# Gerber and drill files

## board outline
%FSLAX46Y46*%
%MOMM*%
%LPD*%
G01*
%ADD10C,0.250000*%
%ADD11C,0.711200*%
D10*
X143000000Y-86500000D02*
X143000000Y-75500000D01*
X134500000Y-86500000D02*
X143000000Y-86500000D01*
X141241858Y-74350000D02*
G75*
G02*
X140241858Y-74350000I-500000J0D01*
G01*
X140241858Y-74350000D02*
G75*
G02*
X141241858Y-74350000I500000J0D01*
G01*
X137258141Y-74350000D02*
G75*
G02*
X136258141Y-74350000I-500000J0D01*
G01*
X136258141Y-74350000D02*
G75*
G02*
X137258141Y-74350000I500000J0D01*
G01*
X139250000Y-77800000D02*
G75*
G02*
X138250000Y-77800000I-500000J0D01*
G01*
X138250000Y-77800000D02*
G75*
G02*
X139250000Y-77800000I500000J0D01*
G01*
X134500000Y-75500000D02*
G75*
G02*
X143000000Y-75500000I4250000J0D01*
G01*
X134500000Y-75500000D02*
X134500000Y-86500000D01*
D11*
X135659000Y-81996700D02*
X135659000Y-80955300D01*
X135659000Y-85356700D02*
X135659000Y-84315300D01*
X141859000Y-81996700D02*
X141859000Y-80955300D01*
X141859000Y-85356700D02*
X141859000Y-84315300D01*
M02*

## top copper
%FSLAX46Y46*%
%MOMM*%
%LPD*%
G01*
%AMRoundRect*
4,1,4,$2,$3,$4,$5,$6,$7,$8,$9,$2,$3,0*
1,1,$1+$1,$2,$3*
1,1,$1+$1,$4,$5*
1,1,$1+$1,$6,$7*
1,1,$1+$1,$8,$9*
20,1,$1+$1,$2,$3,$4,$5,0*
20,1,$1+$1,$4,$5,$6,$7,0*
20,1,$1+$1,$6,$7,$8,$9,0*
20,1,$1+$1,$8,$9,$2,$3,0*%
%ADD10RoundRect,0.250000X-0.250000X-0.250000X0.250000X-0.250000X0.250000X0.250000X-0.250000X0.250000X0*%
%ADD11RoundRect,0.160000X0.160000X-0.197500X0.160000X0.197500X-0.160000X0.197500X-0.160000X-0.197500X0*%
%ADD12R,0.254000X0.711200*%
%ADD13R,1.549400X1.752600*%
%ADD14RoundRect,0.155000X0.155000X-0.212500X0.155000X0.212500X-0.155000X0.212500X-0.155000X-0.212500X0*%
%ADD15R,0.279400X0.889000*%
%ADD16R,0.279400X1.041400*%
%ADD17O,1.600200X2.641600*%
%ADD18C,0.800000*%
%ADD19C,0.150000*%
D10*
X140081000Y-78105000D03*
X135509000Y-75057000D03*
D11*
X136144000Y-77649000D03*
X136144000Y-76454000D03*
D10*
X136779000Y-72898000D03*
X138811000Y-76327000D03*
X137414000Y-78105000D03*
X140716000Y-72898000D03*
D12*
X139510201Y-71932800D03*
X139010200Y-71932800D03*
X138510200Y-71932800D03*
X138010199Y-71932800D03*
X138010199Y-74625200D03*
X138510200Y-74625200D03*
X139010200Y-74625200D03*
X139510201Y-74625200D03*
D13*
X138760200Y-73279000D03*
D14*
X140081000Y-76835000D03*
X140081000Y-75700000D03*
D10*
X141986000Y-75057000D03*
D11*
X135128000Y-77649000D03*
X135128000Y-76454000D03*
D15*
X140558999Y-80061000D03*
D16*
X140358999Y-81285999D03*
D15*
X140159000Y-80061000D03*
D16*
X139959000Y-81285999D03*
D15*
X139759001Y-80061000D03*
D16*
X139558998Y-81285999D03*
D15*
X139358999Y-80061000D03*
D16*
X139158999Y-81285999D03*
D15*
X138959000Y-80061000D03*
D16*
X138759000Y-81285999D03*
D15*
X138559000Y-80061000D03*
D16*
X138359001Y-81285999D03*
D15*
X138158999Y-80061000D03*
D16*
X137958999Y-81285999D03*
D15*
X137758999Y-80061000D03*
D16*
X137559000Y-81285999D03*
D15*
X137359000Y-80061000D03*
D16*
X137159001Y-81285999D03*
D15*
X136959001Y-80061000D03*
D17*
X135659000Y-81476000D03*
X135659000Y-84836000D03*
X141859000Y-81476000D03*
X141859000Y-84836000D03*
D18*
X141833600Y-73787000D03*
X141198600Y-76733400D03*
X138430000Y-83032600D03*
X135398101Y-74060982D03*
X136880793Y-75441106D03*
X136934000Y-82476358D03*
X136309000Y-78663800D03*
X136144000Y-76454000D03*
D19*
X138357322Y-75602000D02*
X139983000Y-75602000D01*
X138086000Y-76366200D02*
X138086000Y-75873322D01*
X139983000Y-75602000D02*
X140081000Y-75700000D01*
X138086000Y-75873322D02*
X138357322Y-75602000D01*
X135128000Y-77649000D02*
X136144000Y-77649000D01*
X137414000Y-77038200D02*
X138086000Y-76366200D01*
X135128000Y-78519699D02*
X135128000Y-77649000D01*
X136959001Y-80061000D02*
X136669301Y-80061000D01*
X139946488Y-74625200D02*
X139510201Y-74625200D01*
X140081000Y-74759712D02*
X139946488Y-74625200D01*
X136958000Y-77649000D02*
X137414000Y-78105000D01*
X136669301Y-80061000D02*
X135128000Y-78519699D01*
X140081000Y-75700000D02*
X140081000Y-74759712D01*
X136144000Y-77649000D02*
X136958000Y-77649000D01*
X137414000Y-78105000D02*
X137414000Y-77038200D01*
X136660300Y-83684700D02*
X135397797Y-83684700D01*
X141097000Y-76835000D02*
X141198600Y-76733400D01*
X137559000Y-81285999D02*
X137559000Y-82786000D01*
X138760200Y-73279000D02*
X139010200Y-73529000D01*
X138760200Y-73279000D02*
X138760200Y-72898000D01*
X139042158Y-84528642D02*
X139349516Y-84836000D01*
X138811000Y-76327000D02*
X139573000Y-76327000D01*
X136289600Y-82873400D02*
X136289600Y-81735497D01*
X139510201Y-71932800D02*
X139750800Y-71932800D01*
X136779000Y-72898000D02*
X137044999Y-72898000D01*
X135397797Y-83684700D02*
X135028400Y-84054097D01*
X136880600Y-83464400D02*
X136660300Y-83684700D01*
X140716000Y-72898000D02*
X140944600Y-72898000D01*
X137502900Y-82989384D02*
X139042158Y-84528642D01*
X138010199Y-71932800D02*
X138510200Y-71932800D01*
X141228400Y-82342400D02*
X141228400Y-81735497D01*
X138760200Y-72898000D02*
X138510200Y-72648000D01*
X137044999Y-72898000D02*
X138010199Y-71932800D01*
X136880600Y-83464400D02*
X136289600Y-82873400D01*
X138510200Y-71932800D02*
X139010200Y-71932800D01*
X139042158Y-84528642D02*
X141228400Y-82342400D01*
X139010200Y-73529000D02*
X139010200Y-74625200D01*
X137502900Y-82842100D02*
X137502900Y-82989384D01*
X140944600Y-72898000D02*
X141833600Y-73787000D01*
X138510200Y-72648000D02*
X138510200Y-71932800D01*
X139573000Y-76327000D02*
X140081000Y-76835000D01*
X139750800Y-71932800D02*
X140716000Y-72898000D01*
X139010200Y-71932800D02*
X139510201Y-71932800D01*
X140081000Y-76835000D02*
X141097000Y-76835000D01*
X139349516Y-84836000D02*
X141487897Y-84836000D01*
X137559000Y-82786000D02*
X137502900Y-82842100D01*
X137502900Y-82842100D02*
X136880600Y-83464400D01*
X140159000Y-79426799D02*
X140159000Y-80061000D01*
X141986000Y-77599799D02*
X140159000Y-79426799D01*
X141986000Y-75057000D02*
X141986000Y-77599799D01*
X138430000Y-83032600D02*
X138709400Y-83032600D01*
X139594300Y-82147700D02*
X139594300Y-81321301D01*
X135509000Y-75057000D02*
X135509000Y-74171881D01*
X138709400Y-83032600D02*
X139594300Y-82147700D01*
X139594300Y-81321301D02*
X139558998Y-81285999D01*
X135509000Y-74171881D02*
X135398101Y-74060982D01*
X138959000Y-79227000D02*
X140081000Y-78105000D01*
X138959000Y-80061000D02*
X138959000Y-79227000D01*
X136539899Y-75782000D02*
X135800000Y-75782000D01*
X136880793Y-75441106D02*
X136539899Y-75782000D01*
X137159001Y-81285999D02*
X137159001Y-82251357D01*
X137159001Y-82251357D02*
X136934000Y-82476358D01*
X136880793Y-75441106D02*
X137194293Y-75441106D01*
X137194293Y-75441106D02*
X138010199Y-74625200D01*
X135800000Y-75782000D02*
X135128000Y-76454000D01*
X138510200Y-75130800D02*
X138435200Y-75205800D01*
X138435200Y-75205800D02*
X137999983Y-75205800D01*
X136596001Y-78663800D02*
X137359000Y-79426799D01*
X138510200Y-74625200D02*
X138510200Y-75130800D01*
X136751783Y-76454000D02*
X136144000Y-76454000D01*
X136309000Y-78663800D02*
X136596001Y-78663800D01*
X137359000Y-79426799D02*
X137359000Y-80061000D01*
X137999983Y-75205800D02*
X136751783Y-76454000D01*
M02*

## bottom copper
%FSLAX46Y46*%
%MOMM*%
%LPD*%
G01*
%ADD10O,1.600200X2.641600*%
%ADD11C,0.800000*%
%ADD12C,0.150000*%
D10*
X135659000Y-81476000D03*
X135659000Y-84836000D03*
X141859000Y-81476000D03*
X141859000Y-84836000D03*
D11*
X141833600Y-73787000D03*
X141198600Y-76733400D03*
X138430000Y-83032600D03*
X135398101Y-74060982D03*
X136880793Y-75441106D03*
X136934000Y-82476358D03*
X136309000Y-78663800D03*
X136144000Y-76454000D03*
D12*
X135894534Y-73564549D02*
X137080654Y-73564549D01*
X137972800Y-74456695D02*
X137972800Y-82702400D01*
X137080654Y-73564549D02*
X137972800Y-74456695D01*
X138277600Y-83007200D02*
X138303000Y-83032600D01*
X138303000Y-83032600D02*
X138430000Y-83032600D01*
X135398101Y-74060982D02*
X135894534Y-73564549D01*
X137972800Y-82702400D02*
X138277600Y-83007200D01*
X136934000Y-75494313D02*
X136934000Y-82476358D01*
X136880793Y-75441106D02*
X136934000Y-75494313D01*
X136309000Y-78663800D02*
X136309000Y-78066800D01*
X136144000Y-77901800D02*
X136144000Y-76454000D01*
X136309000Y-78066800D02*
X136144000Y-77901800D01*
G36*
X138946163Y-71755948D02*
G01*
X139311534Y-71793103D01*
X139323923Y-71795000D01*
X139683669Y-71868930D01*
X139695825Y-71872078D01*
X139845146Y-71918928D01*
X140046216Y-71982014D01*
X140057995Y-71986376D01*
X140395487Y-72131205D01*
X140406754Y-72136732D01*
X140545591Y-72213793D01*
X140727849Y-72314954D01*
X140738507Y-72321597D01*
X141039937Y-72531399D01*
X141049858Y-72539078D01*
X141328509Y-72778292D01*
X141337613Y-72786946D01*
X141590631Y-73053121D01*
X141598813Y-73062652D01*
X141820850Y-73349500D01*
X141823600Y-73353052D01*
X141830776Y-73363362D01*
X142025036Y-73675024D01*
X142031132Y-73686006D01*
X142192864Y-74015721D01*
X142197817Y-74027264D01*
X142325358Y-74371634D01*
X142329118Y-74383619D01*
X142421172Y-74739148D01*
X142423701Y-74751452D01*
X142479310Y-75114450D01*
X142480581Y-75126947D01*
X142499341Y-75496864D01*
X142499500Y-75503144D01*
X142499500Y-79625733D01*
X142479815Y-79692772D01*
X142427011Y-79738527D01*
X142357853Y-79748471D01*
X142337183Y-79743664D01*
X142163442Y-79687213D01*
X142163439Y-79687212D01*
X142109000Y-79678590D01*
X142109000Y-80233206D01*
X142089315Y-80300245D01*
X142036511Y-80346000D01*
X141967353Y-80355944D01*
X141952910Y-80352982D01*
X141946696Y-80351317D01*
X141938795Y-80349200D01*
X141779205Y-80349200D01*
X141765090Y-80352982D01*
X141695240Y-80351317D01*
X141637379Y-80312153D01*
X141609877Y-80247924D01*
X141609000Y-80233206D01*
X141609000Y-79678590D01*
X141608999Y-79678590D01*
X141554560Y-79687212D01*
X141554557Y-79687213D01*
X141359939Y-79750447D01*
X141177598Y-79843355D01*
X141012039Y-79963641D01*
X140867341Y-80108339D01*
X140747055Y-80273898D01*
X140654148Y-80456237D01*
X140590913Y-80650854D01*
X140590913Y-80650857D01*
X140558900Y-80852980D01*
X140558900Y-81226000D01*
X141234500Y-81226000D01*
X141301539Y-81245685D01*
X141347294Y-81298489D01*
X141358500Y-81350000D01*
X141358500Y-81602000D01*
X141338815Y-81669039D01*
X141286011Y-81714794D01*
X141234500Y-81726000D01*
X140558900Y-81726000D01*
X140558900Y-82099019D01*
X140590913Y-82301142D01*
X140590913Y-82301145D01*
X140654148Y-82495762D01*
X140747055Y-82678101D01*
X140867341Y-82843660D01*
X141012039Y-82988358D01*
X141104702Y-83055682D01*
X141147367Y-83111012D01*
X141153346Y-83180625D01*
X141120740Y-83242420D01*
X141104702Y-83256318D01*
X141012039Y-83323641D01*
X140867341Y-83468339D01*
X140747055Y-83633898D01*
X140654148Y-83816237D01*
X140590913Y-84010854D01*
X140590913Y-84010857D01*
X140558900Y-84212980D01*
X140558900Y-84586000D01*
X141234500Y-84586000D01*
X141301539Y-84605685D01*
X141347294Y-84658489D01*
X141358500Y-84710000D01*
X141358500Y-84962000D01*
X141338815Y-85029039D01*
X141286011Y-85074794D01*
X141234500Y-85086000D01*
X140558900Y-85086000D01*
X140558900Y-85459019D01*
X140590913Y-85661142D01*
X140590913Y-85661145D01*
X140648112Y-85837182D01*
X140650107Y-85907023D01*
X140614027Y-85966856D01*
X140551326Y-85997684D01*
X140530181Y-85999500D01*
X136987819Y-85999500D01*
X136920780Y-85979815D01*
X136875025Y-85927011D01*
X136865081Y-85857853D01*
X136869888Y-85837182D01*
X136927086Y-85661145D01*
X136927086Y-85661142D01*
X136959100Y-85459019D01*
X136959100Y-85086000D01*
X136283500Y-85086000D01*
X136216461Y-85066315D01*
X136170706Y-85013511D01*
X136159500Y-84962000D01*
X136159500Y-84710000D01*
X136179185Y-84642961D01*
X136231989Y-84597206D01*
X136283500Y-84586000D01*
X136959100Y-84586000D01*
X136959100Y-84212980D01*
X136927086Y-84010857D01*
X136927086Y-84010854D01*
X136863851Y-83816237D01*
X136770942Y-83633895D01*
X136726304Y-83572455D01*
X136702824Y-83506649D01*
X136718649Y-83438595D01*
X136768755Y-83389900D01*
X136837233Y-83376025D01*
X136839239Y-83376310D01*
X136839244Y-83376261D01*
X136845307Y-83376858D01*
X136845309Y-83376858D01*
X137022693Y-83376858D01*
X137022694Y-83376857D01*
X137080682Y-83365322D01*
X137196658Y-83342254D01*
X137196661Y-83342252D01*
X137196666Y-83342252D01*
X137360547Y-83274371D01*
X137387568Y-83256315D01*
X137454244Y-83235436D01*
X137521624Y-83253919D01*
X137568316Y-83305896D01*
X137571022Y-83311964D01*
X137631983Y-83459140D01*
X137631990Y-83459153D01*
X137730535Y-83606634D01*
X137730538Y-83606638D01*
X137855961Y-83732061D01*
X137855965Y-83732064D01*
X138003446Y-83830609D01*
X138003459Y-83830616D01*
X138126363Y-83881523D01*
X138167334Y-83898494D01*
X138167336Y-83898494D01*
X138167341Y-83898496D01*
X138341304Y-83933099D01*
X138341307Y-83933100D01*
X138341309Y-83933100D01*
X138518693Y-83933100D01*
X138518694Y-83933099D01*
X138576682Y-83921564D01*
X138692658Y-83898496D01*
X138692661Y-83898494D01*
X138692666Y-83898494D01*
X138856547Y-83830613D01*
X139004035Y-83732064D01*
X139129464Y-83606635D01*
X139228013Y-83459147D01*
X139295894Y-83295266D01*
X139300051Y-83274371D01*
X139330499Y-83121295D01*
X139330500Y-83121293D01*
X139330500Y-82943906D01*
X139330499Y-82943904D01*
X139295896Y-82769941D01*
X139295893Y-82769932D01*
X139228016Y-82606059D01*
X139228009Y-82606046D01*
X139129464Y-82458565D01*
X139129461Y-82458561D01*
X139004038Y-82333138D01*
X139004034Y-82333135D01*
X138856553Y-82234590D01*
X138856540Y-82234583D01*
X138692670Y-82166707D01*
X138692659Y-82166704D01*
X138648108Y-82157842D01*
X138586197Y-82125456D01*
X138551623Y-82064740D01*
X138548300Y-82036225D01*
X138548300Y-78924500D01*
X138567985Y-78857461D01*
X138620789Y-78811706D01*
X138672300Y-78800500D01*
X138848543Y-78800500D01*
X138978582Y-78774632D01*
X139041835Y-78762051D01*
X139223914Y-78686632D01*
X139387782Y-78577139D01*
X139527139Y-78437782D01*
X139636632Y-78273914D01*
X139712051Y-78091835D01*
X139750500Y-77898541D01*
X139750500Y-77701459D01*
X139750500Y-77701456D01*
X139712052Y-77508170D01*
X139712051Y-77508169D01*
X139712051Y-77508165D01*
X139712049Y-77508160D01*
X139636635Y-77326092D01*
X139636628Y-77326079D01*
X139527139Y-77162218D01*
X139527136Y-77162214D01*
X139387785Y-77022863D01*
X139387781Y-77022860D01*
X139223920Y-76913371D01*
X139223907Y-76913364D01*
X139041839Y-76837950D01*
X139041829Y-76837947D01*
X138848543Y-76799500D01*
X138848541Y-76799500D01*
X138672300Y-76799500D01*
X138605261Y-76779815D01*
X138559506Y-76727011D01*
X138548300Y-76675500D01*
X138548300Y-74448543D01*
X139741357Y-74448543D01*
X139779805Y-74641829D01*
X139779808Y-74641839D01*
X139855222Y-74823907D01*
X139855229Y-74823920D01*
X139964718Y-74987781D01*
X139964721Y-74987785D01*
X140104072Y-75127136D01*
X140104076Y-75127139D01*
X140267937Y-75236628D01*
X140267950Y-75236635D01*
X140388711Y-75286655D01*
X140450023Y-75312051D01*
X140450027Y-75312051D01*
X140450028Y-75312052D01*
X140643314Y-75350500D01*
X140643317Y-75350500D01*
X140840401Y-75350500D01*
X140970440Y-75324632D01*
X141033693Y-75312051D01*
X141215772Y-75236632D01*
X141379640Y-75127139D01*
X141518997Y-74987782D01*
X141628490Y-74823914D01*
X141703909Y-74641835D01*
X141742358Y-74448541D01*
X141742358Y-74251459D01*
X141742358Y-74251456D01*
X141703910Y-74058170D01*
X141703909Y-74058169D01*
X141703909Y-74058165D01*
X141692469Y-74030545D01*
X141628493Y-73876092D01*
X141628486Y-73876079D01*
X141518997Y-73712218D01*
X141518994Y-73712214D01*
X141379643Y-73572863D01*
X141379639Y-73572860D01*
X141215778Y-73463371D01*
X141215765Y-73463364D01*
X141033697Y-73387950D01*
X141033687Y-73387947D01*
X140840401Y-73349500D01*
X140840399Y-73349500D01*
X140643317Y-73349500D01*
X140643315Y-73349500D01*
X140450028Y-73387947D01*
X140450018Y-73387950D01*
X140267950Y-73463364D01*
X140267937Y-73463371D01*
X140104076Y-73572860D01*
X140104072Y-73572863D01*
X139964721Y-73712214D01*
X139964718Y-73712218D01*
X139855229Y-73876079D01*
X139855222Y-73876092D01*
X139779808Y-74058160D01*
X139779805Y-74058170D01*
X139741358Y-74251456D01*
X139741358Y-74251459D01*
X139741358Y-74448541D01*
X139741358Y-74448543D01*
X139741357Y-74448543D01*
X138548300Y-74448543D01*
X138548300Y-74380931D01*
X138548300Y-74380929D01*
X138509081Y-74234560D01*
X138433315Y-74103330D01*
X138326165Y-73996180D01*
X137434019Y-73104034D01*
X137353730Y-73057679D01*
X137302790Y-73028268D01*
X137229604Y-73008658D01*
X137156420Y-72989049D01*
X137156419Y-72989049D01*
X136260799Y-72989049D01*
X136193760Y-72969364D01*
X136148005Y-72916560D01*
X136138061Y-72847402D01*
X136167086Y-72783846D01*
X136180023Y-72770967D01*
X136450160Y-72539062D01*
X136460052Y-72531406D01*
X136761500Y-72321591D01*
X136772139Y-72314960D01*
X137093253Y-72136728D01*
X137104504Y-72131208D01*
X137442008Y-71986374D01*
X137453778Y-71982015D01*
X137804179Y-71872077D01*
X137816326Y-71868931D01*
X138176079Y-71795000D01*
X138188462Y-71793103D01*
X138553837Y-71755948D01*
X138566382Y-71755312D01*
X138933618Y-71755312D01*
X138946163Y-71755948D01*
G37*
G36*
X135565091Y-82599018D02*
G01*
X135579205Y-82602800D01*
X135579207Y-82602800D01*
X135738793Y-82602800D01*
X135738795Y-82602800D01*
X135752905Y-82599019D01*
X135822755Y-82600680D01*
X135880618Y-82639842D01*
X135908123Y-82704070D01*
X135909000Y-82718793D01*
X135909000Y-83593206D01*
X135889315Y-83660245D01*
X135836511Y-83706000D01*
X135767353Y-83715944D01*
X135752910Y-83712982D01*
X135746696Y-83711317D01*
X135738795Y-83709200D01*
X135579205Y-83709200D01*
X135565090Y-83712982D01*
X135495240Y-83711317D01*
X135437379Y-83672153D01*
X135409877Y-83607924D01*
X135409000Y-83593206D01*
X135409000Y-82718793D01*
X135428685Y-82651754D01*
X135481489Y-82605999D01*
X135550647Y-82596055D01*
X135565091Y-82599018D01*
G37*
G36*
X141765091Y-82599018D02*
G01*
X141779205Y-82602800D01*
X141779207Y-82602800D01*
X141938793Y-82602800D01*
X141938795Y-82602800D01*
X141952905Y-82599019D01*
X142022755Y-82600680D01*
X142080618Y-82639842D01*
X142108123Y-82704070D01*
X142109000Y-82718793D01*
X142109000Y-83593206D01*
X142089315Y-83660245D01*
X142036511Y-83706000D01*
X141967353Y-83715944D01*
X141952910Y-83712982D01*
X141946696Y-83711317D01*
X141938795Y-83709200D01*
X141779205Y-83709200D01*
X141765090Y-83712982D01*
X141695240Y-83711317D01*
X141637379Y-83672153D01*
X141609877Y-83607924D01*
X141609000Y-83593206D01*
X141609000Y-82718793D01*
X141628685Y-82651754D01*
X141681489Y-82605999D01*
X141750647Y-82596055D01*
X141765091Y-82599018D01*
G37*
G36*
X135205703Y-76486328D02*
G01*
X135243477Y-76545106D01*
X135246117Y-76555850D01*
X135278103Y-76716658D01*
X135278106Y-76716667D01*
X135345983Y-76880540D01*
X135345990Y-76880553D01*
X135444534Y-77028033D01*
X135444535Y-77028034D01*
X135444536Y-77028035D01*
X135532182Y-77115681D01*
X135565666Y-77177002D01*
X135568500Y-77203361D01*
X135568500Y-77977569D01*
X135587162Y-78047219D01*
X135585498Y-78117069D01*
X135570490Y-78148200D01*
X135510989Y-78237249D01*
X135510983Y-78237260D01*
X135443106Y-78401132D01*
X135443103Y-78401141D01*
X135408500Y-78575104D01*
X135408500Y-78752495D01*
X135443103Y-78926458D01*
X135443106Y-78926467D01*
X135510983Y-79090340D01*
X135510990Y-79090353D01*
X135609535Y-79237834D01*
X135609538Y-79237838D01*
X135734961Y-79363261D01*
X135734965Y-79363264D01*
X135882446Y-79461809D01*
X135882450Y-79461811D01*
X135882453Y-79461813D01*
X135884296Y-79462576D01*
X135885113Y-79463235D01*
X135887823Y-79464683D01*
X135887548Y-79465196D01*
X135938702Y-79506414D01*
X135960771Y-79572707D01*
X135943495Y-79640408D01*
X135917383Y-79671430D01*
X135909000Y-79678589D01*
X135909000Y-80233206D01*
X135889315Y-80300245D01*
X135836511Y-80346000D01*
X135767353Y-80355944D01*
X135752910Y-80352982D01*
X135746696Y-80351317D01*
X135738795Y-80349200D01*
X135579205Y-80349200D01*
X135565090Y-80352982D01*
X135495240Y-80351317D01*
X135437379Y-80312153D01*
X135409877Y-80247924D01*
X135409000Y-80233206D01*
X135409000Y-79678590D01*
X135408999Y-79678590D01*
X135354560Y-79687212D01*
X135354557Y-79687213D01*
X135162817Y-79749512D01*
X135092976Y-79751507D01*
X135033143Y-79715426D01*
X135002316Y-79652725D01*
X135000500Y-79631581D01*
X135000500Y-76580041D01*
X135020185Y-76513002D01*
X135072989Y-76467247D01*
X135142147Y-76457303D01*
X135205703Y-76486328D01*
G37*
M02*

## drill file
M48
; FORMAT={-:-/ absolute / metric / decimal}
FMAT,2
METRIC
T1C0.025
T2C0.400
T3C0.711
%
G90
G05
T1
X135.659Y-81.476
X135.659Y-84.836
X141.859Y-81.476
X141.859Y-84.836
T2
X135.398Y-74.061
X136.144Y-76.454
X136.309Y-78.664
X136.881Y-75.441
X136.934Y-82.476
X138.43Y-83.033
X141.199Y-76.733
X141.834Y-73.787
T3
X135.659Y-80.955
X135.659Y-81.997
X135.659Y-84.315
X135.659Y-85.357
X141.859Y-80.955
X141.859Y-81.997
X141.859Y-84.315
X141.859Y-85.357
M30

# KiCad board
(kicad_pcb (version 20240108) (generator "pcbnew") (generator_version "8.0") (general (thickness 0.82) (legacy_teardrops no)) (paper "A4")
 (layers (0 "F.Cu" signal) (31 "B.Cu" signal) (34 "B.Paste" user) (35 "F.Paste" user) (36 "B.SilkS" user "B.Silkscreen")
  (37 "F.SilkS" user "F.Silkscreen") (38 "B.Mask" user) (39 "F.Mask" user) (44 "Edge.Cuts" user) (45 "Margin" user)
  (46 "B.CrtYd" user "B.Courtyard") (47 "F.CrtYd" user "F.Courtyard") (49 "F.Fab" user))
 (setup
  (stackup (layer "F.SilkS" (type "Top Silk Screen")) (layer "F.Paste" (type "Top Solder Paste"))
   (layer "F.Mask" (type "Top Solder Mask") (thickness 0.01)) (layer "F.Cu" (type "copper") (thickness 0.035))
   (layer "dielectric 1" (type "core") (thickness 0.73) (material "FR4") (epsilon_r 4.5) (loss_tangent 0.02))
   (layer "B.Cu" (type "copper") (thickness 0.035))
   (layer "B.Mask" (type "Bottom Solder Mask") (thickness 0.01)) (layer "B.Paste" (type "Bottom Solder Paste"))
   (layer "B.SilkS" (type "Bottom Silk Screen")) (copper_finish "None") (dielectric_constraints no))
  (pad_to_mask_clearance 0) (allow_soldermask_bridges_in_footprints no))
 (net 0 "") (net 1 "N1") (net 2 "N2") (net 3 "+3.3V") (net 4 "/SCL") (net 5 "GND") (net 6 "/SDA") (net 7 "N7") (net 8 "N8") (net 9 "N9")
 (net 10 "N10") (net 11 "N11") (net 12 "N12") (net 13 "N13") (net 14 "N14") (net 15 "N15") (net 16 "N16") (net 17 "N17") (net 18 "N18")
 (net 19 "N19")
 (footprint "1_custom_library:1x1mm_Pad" (layer "F.Cu") (at 140.081 78.105)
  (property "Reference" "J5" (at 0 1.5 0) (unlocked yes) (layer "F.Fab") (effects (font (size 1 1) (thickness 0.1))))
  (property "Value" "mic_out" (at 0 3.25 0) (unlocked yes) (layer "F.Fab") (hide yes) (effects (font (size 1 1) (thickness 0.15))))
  (pad "1" smd roundrect (at 0 0) (size 1 1) (layers "F.Cu" "F.Mask") (roundrect_rratio 0.25) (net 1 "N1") (thermal_bridge_angle 45)))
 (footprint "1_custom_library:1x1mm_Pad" (layer "F.Cu") (at 135.509 75.057)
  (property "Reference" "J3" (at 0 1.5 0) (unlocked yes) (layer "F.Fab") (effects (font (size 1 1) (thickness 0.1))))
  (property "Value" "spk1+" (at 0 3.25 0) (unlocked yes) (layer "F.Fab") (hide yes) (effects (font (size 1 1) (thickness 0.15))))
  (pad "1" smd roundrect (at 0 0) (size 1 1) (layers "F.Cu" "F.Mask") (roundrect_rratio 0.25) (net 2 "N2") (thermal_bridge_angle 45)))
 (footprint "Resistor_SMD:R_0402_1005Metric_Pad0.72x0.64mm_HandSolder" (layer "F.Cu") (at 136.144 77.0515 90)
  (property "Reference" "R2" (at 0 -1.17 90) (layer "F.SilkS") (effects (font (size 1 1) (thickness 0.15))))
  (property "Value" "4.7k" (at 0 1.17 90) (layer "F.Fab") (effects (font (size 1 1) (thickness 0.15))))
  (pad "1" smd roundrect (at -0.5975 0 90) (size 0.715 0.64) (layers "F.Cu" "F.Paste" "F.Mask") (roundrect_rratio 0.25) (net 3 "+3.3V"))
  (pad "2" smd roundrect (at 0.5975 0 90) (size 0.715 0.64) (layers "F.Cu" "F.Paste" "F.Mask") (roundrect_rratio 0.25) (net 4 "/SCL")))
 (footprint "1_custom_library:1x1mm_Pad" (layer "F.Cu") (at 136.779 72.898)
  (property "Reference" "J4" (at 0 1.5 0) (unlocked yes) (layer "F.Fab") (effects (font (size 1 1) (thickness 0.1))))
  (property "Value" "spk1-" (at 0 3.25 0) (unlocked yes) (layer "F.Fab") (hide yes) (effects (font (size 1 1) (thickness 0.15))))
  (pad "1" smd roundrect (at 0 0) (size 1 1) (layers "F.Cu" "F.Mask") (roundrect_rratio 0.25) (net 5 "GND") (thermal_bridge_angle 45)))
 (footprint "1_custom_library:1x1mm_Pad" (layer "F.Cu") (at 138.811 76.327)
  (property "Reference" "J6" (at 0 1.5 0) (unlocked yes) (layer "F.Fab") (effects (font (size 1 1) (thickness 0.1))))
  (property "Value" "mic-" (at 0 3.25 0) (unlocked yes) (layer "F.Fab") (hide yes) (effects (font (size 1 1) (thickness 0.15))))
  (pad "1" smd roundrect (at 0 0) (size 1 1) (layers "F.Cu" "F.Mask") (roundrect_rratio 0.25) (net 5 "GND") (thermal_bridge_angle 45)))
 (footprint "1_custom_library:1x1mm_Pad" (layer "F.Cu") (at 137.414 78.105)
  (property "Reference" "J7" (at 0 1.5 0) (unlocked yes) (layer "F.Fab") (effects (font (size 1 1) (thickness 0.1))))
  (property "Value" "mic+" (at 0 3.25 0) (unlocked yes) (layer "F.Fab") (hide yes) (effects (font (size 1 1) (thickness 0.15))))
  (pad "1" smd roundrect (at 0 0) (size 1 1) (layers "F.Cu" "F.Mask") (roundrect_rratio 0.25) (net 3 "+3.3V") (thermal_bridge_angle 45)))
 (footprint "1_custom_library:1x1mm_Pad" (layer "F.Cu") (at 140.716 72.898)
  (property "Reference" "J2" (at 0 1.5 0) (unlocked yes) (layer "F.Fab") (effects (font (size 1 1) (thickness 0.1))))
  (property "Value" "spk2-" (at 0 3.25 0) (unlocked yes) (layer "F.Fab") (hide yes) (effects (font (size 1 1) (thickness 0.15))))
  (pad "1" smd roundrect (at 0 0) (size 1 1) (layers "F.Cu" "F.Mask") (roundrect_rratio 0.25) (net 5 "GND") (thermal_bridge_angle 45)))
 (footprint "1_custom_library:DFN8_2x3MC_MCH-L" (layer "F.Cu") (at 138.7602 73.279 -90)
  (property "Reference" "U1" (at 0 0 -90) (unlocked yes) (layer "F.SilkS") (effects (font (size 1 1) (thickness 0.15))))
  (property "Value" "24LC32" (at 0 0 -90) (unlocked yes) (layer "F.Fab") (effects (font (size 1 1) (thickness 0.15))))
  (pad "1" smd rect (at -1.3462 -0.750001 270) (size 0.7112 0.254) (layers "F.Cu" "F.Paste" "F.Mask") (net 5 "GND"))
  (pad "2" smd rect (at -1.3462 -0.25 270) (size 0.7112 0.254) (layers "F.Cu" "F.Paste" "F.Mask") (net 5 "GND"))
  (pad "3" smd rect (at -1.3462 0.25 270) (size 0.7112 0.254) (layers "F.Cu" "F.Paste" "F.Mask") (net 5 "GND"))
  (pad "4" smd rect (at -1.3462 0.750001 270) (size 0.7112 0.254) (layers "F.Cu" "F.Paste" "F.Mask") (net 5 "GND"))
  (pad "5" smd rect (at 1.3462 0.750001 270) (size 0.7112 0.254) (layers "F.Cu" "F.Paste" "F.Mask") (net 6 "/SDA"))
  (pad "6" smd rect (at 1.3462 0.25 270) (size 0.7112 0.254) (layers "F.Cu" "F.Paste" "F.Mask") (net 4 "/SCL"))
  (pad "7" smd rect (at 1.3462 -0.25 270) (size 0.7112 0.254) (layers "F.Cu" "F.Paste" "F.Mask") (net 5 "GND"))
  (pad "8" smd rect (at 1.3462 -0.750001 270) (size 0.7112 0.254) (layers "F.Cu" "F.Paste" "F.Mask") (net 3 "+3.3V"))
  (pad "9" smd rect (at 0 0 270) (size 1.7526 1.5494) (layers "F.Cu" "F.Paste" "F.Mask") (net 5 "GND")))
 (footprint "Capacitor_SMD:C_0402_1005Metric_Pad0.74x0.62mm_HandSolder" (layer "F.Cu") (at 140.081 76.2675 90)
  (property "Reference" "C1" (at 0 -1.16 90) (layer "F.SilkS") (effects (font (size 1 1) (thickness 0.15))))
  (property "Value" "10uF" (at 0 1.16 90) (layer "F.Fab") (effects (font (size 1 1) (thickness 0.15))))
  (pad "1" smd roundrect (at -0.5675 0 90) (size 0.735 0.62) (layers "F.Cu" "F.Paste" "F.Mask") (roundrect_rratio 0.25) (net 5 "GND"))
  (pad "2" smd roundrect (at 0.5675 0 90) (size 0.735 0.62) (layers "F.Cu" "F.Paste" "F.Mask") (roundrect_rratio 0.25) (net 3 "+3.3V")))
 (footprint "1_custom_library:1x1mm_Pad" (layer "F.Cu") (at 141.986 75.057)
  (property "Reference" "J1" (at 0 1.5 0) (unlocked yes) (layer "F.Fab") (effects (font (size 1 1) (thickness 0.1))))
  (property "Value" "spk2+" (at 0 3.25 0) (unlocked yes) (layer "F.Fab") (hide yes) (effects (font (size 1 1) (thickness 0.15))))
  (pad "1" smd roundrect (at 0 0) (size 1 1) (layers "F.Cu" "F.Mask") (roundrect_rratio 0.25) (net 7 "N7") (thermal_bridge_angle 45)))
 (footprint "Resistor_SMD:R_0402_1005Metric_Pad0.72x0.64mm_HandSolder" (layer "F.Cu") (at 135.128 77.0515 90)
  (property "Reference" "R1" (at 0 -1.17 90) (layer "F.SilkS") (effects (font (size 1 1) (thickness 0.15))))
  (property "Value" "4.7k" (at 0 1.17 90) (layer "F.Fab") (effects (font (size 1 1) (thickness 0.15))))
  (pad "1" smd roundrect (at -0.5975 0 90) (size 0.715 0.64) (layers "F.Cu" "F.Paste" "F.Mask") (roundrect_rratio 0.25) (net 3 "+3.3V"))
  (pad "2" smd roundrect (at 0.5975 0 90) (size 0.715 0.64) (layers "F.Cu" "F.Paste" "F.Mask") (roundrect_rratio 0.25) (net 6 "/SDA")))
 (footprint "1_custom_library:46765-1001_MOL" (layer "F.Cu") (at 138.759 83.3841)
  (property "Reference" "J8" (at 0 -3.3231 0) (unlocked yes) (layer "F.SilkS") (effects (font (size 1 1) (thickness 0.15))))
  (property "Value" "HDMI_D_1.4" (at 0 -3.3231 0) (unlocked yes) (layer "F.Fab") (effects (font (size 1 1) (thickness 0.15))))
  (fp_line (start -3.1 -1.3874) (end -3.1 -2.4288) (stroke (width 0.7112) (type solid)) (layer "Edge.Cuts"))
  (fp_line (start -3.1 1.9726) (end -3.1 0.9312) (stroke (width 0.7112) (type solid)) (layer "Edge.Cuts"))
  (fp_line (start 3.1 -1.3874) (end 3.1 -2.4288) (stroke (width 0.7112) (type solid)) (layer "Edge.Cuts"))
  (fp_line (start 3.1 1.9726) (end 3.1 0.9312) (stroke (width 0.7112) (type solid)) (layer "Edge.Cuts"))
  (pad "" np_thru_hole circle (at -3.1 -2.4288) (size 0.7112 0.7112) (drill 0.7112) (layers "*.Cu" "*.Mask"))
  (pad "" np_thru_hole circle (at -3.1 -1.3874) (size 0.7112 0.7112) (drill 0.7112) (layers "*.Cu" "*.Mask"))
  (pad "" np_thru_hole circle (at -3.1 0.9312) (size 0.7112 0.7112) (drill 0.7112) (layers "*.Cu" "*.Mask"))
  (pad "" np_thru_hole circle (at -3.1 1.9726) (size 0.7112 0.7112) (drill 0.7112) (layers "*.Cu" "*.Mask"))
  (pad "" np_thru_hole circle (at 3.1 -2.4288) (size 0.7112 0.7112) (drill 0.7112) (layers "*.Cu" "*.Mask"))
  (pad "" np_thru_hole circle (at 3.1 -1.3874) (size 0.7112 0.7112) (drill 0.7112) (layers "*.Cu" "*.Mask"))
  (pad "" np_thru_hole circle (at 3.1 0.9312) (size 0.7112 0.7112) (drill 0.7112) (layers "*.Cu" "*.Mask"))
  (pad "" np_thru_hole circle (at 3.1 1.9726) (size 0.7112 0.7112) (drill 0.7112) (layers "*.Cu" "*.Mask"))
  (pad "1" smd rect (at 1.799999 -3.3231) (size 0.2794 0.889) (layers "F.Cu" "F.Paste" "F.Mask") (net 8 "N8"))
  (pad "2" smd rect (at 1.599999 -2.098101) (size 0.2794 1.0414) (layers "F.Cu" "F.Paste" "F.Mask") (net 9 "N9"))
  (pad "3" smd rect (at 1.4 -3.3231) (size 0.2794 0.889) (layers "F.Cu" "F.Paste" "F.Mask") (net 7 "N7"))
  (pad "4" smd rect (at 1.2 -2.098101) (size 0.2794 1.0414) (layers "F.Cu" "F.Paste" "F.Mask") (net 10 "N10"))
  (pad "5" smd rect (at 1.000001 -3.3231) (size 0.2794 0.889) (layers "F.Cu" "F.Paste" "F.Mask") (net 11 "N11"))
  (pad "6" smd rect (at 0.799998 -2.098101) (size 0.2794 1.0414) (layers "F.Cu" "F.Paste" "F.Mask") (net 2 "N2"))
  (pad "7" smd rect (at 0.599999 -3.3231) (size 0.2794 0.889) (layers "F.Cu" "F.Paste" "F.Mask") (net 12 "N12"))
  (pad "8" smd rect (at 0.399999 -2.098101) (size 0.2794 1.0414) (layers "F.Cu" "F.Paste" "F.Mask") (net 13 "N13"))
  (pad "9" smd rect (at 0.2 -3.3231) (size 0.2794 0.889) (layers "F.Cu" "F.Paste" "F.Mask") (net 1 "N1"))
  (pad "10" smd rect (at 0 -2.098101) (size 0.2794 1.0414) (layers "F.Cu" "F.Paste" "F.Mask") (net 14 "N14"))
  (pad "11" smd rect (at -0.2 -3.3231) (size 0.2794 0.889) (layers "F.Cu" "F.Paste" "F.Mask") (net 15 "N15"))
  (pad "12" smd rect (at -0.399999 -2.098101) (size 0.2794 1.0414) (layers "F.Cu" "F.Paste" "F.Mask") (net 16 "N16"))
  (pad "13" smd rect (at -0.600001 -3.3231) (size 0.2794 0.889) (layers "F.Cu" "F.Paste" "F.Mask") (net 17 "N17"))
  (pad "14" smd rect (at -0.800001 -2.098101) (size 0.2794 1.0414) (layers "F.Cu" "F.Paste" "F.Mask") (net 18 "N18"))
  (pad "15" smd rect (at -1.000001 -3.3231) (size 0.2794 0.889) (layers "F.Cu" "F.Paste" "F.Mask") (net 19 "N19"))
  (pad "16" smd rect (at -1.2 -2.098101) (size 0.2794 1.0414) (layers "F.Cu" "F.Paste" "F.Mask") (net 5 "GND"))
  (pad "17" smd rect (at -1.4 -3.3231) (size 0.2794 0.889) (layers "F.Cu" "F.Paste" "F.Mask") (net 4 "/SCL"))
  (pad "18" smd rect (at -1.599999 -2.098101) (size 0.2794 1.0414) (layers "F.Cu" "F.Paste" "F.Mask") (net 6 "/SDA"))
  (pad "19" smd rect (at -1.799999 -3.3231) (size 0.2794 0.889) (layers "F.Cu" "F.Paste" "F.Mask") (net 3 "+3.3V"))
  (pad "SH" thru_hole oval (at -3.1 -1.9081 90) (size 2.6416 1.6002) (drill 0.0254) (layers "*.Cu" "*.Mask") (remove_unused_layers no)
   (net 5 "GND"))
  (pad "SH" thru_hole oval (at -3.1 1.4519 90) (size 2.6416 1.6002) (drill 0.0254) (layers "*.Cu" "*.Mask") (remove_unused_layers no)
   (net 5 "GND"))
  (pad "SH" thru_hole oval (at 3.1 -1.9081 90) (size 2.6416 1.6002) (drill 0.0254) (layers "*.Cu" "*.Mask") (remove_unused_layers no)
   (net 5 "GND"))
  (pad "SH" thru_hole oval (at 3.1 1.4519 90) (size 2.6416 1.6002) (drill 0.0254) (layers "*.Cu" "*.Mask") (remove_unused_layers no)
   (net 5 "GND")))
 (gr_line (start 143 86.5) (end 143 75.5) (stroke (width 0.25) (type default)) (layer "Edge.Cuts"))
 (gr_line (start 134.5 86.5) (end 143 86.5) (stroke (width 0.25) (type default)) (layer "Edge.Cuts"))
 (gr_circle (center 140.741858 74.35) (end 141.241858 74.35) (stroke (width 0.25) (type default)) (fill none) (layer "Edge.Cuts"))
 (gr_circle (center 136.758141 74.35) (end 137.258141 74.35) (stroke (width 0.25) (type default)) (fill none) (layer "Edge.Cuts"))
 (gr_circle (center 138.75 77.8) (end 139.25 77.8) (stroke (width 0.25) (type default)) (fill none) (layer "Edge.Cuts"))
 (gr_arc (start 134.5 75.5) (mid 138.75 71.25) (end 143 75.5) (stroke (width 0.25) (type default)) (layer "Edge.Cuts"))
 (gr_line (start 134.5 75.5) (end 134.5 86.5) (stroke (width 0.25) (type default)) (layer "Edge.Cuts"))
 (segment (start 138.357322 75.602) (end 139.983 75.602) (width 0.15) (layer "F.Cu") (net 3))
 (segment (start 138.086 76.3662) (end 138.086 75.873322) (width 0.15) (layer "F.Cu") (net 3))
 (segment (start 139.983 75.602) (end 140.081 75.7) (width 0.15) (layer "F.Cu") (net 3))
 (segment (start 138.086 75.873322) (end 138.357322 75.602) (width 0.15) (layer "F.Cu") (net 3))
 (segment (start 135.128 77.649) (end 136.144 77.649) (width 0.15) (layer "F.Cu") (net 3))
 (segment (start 137.414 77.0382) (end 138.086 76.3662) (width 0.15) (layer "F.Cu") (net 3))
 (segment (start 135.128 78.519699) (end 135.128 77.649) (width 0.15) (layer "F.Cu") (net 3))
 (segment (start 136.959001 80.061) (end 136.669301 80.061) (width 0.15) (layer "F.Cu") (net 3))
 (segment (start 139.946488 74.6252) (end 139.510201 74.6252) (width 0.15) (layer "F.Cu") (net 3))
 (segment (start 140.081 74.759712) (end 139.946488 74.6252) (width 0.15) (layer "F.Cu") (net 3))
 (segment (start 136.958 77.649) (end 137.414 78.105) (width 0.15) (layer "F.Cu") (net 3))
 (segment (start 136.669301 80.061) (end 135.128 78.519699) (width 0.15) (layer "F.Cu") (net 3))
 (segment (start 140.081 75.7) (end 140.081 74.759712) (width 0.15) (layer "F.Cu") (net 3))
 (segment (start 136.144 77.649) (end 136.958 77.649) (width 0.15) (layer "F.Cu") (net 3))
 (segment (start 137.414 78.105) (end 137.414 77.0382) (width 0.15) (layer "F.Cu") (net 3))
 (segment (start 136.6603 83.6847) (end 135.397797 83.6847) (width 0.15) (layer "F.Cu") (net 5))
 (segment (start 141.097 76.835) (end 141.1986 76.7334) (width 0.15) (layer "F.Cu") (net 5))
 (segment (start 137.559 81.285999) (end 137.559 82.786) (width 0.15) (layer "F.Cu") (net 5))
 (segment (start 138.7602 73.279) (end 139.0102 73.529) (width 0.15) (layer "F.Cu") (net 5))
 (segment (start 138.7602 73.279) (end 138.7602 72.898) (width 0.15) (layer "F.Cu") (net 5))
 (segment (start 139.042158 84.528642) (end 139.349516 84.836) (width 0.15) (layer "F.Cu") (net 5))
 (segment (start 138.811 76.327) (end 139.573 76.327) (width 0.15) (layer "F.Cu") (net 5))
 (segment (start 136.2896 82.8734) (end 136.2896 81.735497) (width 0.15) (layer "F.Cu") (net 5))
 (segment (start 139.510201 71.9328) (end 139.7508 71.9328) (width 0.15) (layer "F.Cu") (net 5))
 (segment (start 136.779 72.898) (end 137.044999 72.898) (width 0.15) (layer "F.Cu") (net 5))
 (segment (start 135.397797 83.6847) (end 135.0284 84.054097) (width 0.15) (layer "F.Cu") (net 5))
 (segment (start 136.8806 83.4644) (end 136.6603 83.6847) (width 0.15) (layer "F.Cu") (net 5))
 (segment (start 140.716 72.898) (end 140.9446 72.898) (width 0.15) (layer "F.Cu") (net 5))
 (segment (start 137.5029 82.989384) (end 139.042158 84.528642) (width 0.15) (layer "F.Cu") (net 5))
 (segment (start 138.010199 71.9328) (end 138.5102 71.9328) (width 0.15) (layer "F.Cu") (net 5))
 (segment (start 141.2284 82.3424) (end 141.2284 81.735497) (width 0.15) (layer "F.Cu") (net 5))
 (segment (start 138.7602 72.898) (end 138.5102 72.648) (width 0.15) (layer "F.Cu") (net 5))
 (segment (start 137.044999 72.898) (end 138.010199 71.9328) (width 0.15) (layer "F.Cu") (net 5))
 (segment (start 136.8806 83.4644) (end 136.2896 82.8734) (width 0.15) (layer "F.Cu") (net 5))
 (segment (start 138.5102 71.9328) (end 139.0102 71.9328) (width 0.15) (layer "F.Cu") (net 5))
 (segment (start 139.042158 84.528642) (end 141.2284 82.3424) (width 0.15) (layer "F.Cu") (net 5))
 (segment (start 139.0102 73.529) (end 139.0102 74.6252) (width 0.15) (layer "F.Cu") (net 5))
 (segment (start 137.5029 82.8421) (end 137.5029 82.989384) (width 0.15) (layer "F.Cu") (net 5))
 (segment (start 140.9446 72.898) (end 141.8336 73.787) (width 0.15) (layer "F.Cu") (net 5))
 (segment (start 138.5102 72.648) (end 138.5102 71.9328) (width 0.15) (layer "F.Cu") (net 5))
 (segment (start 139.573 76.327) (end 140.081 76.835) (width 0.15) (layer "F.Cu") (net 5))
 (segment (start 139.7508 71.9328) (end 140.716 72.898) (width 0.15) (layer "F.Cu") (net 5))
 (segment (start 139.0102 71.9328) (end 139.510201 71.9328) (width 0.15) (layer "F.Cu") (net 5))
 (segment (start 140.081 76.835) (end 141.097 76.835) (width 0.15) (layer "F.Cu") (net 5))
 (segment (start 139.349516 84.836) (end 141.487897 84.836) (width 0.15) (layer "F.Cu") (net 5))
 (segment (start 137.559 82.786) (end 137.5029 82.8421) (width 0.15) (layer "F.Cu") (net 5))
 (segment (start 137.5029 82.8421) (end 136.8806 83.4644) (width 0.15) (layer "F.Cu") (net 5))
 (via (at 141.8336 73.787) (size 0.8) (drill 0.4) (layers "F.Cu" "B.Cu") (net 5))
 (via (at 141.1986 76.7334) (size 0.8) (drill 0.4) (layers "F.Cu" "B.Cu") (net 5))
 (segment (start 140.159 79.426799) (end 140.159 80.061) (width 0.15) (layer "F.Cu") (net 7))
 (segment (start 141.986 77.599799) (end 140.159 79.426799) (width 0.15) (layer "F.Cu") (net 7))
 (segment (start 141.986 75.057) (end 141.986 77.599799) (width 0.15) (layer "F.Cu") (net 7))
 (segment (start 138.43 83.0326) (end 138.7094 83.0326) (width 0.15) (layer "F.Cu") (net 2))
 (segment (start 139.5943 82.1477) (end 139.5943 81.321301) (width 0.15) (layer "F.Cu") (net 2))
 (segment (start 135.509 75.057) (end 135.509 74.171881) (width 0.15) (layer "F.Cu") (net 2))
 (segment (start 138.7094 83.0326) (end 139.5943 82.1477) (width 0.15) (layer "F.Cu") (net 2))
 (segment (start 139.5943 81.321301) (end 139.558998 81.285999) (width 0.15) (layer "F.Cu") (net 2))
 (segment (start 135.509 74.171881) (end 135.398101 74.060982) (width 0.15) (layer "F.Cu") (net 2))
 (via (at 138.43 83.0326) (size 0.8) (drill 0.4) (layers "F.Cu" "B.Cu") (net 2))
 (via (at 135.398101 74.060982) (size 0.8) (drill 0.4) (layers "F.Cu" "B.Cu") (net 2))
 (segment (start 135.894534 73.564549) (end 137.080654 73.564549) (width 0.15) (layer "B.Cu") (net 2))
 (segment (start 137.9728 74.456695) (end 137.9728 82.7024) (width 0.15) (layer "B.Cu") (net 2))
 (segment (start 137.080654 73.564549) (end 137.9728 74.456695) (width 0.15) (layer "B.Cu") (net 2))
 (segment (start 138.2776 83.0072) (end 138.303 83.0326) (width 0.15) (layer "B.Cu") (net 2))
 (segment (start 138.303 83.0326) (end 138.43 83.0326) (width 0.15) (layer "B.Cu") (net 2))
 (segment (start 135.398101 74.060982) (end 135.894534 73.564549) (width 0.15) (layer "B.Cu") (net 2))
 (segment (start 137.9728 82.7024) (end 138.2776 83.0072) (width 0.15) (layer "B.Cu") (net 2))
 (segment (start 138.959 79.227) (end 140.081 78.105) (width 0.15) (layer "F.Cu") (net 1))
 (segment (start 138.959 80.061) (end 138.959 79.227) (width 0.15) (layer "F.Cu") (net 1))
 (segment (start 136.539899 75.782) (end 135.8 75.782) (width 0.15) (layer "F.Cu") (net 6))
 (segment (start 136.880793 75.441106) (end 136.539899 75.782) (width 0.15) (layer "F.Cu") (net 6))
 (segment (start 137.159001 81.285999) (end 137.159001 82.251357) (width 0.15) (layer "F.Cu") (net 6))
 (segment (start 137.159001 82.251357) (end 136.934 82.476358) (width 0.15) (layer "F.Cu") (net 6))
 (segment (start 136.880793 75.441106) (end 137.194293 75.441106) (width 0.15) (layer "F.Cu") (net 6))
 (segment (start 137.194293 75.441106) (end 138.010199 74.6252) (width 0.15) (layer "F.Cu") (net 6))
 (segment (start 135.8 75.782) (end 135.128 76.454) (width 0.15) (layer "F.Cu") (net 6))
 (via (at 136.880793 75.441106) (size 0.8) (drill 0.4) (layers "F.Cu" "B.Cu") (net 6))
 (via (at 136.934 82.476358) (size 0.8) (drill 0.4) (layers "F.Cu" "B.Cu") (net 6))
 (segment (start 136.934 75.494313) (end 136.934 82.476358) (width 0.15) (layer "B.Cu") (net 6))
 (segment (start 136.880793 75.441106) (end 136.934 75.494313) (width 0.15) (layer "B.Cu") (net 6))
 (segment (start 138.5102 75.1308) (end 138.4352 75.2058) (width 0.15) (layer "F.Cu") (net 4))
 (segment (start 138.4352 75.2058) (end 137.999983 75.2058) (width 0.15) (layer "F.Cu") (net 4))
 (segment (start 136.596001 78.6638) (end 137.359 79.426799) (width 0.15) (layer "F.Cu") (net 4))
 (segment (start 138.5102 74.6252) (end 138.5102 75.1308) (width 0.15) (layer "F.Cu") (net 4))
 (segment (start 136.751783 76.454) (end 136.144 76.454) (width 0.15) (layer "F.Cu") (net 4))
 (segment (start 136.309 78.6638) (end 136.596001 78.6638) (width 0.15) (layer "F.Cu") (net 4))
 (segment (start 137.359 79.426799) (end 137.359 80.061) (width 0.15) (layer "F.Cu") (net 4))
 (segment (start 137.999983 75.2058) (end 136.751783 76.454) (width 0.15) (layer "F.Cu") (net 4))
 (via (at 136.309 78.6638) (size 0.8) (drill 0.4) (layers "F.Cu" "B.Cu") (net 4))
 (via (at 136.144 76.454) (size 0.8) (drill 0.4) (layers "F.Cu" "B.Cu") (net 4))
 (segment (start 136.309 78.6638) (end 136.309 78.0668) (width 0.15) (layer "B.Cu") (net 4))
 (segment (start 136.144 77.9018) (end 136.144 76.454) (width 0.15) (layer "B.Cu") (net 4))
 (segment (start 136.309 78.0668) (end 136.144 77.9018) (width 0.15) (layer "B.Cu") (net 4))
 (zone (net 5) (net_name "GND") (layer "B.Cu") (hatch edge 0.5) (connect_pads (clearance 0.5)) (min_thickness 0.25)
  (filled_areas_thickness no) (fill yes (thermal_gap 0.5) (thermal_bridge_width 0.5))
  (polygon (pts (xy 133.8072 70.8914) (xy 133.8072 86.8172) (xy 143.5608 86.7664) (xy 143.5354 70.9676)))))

